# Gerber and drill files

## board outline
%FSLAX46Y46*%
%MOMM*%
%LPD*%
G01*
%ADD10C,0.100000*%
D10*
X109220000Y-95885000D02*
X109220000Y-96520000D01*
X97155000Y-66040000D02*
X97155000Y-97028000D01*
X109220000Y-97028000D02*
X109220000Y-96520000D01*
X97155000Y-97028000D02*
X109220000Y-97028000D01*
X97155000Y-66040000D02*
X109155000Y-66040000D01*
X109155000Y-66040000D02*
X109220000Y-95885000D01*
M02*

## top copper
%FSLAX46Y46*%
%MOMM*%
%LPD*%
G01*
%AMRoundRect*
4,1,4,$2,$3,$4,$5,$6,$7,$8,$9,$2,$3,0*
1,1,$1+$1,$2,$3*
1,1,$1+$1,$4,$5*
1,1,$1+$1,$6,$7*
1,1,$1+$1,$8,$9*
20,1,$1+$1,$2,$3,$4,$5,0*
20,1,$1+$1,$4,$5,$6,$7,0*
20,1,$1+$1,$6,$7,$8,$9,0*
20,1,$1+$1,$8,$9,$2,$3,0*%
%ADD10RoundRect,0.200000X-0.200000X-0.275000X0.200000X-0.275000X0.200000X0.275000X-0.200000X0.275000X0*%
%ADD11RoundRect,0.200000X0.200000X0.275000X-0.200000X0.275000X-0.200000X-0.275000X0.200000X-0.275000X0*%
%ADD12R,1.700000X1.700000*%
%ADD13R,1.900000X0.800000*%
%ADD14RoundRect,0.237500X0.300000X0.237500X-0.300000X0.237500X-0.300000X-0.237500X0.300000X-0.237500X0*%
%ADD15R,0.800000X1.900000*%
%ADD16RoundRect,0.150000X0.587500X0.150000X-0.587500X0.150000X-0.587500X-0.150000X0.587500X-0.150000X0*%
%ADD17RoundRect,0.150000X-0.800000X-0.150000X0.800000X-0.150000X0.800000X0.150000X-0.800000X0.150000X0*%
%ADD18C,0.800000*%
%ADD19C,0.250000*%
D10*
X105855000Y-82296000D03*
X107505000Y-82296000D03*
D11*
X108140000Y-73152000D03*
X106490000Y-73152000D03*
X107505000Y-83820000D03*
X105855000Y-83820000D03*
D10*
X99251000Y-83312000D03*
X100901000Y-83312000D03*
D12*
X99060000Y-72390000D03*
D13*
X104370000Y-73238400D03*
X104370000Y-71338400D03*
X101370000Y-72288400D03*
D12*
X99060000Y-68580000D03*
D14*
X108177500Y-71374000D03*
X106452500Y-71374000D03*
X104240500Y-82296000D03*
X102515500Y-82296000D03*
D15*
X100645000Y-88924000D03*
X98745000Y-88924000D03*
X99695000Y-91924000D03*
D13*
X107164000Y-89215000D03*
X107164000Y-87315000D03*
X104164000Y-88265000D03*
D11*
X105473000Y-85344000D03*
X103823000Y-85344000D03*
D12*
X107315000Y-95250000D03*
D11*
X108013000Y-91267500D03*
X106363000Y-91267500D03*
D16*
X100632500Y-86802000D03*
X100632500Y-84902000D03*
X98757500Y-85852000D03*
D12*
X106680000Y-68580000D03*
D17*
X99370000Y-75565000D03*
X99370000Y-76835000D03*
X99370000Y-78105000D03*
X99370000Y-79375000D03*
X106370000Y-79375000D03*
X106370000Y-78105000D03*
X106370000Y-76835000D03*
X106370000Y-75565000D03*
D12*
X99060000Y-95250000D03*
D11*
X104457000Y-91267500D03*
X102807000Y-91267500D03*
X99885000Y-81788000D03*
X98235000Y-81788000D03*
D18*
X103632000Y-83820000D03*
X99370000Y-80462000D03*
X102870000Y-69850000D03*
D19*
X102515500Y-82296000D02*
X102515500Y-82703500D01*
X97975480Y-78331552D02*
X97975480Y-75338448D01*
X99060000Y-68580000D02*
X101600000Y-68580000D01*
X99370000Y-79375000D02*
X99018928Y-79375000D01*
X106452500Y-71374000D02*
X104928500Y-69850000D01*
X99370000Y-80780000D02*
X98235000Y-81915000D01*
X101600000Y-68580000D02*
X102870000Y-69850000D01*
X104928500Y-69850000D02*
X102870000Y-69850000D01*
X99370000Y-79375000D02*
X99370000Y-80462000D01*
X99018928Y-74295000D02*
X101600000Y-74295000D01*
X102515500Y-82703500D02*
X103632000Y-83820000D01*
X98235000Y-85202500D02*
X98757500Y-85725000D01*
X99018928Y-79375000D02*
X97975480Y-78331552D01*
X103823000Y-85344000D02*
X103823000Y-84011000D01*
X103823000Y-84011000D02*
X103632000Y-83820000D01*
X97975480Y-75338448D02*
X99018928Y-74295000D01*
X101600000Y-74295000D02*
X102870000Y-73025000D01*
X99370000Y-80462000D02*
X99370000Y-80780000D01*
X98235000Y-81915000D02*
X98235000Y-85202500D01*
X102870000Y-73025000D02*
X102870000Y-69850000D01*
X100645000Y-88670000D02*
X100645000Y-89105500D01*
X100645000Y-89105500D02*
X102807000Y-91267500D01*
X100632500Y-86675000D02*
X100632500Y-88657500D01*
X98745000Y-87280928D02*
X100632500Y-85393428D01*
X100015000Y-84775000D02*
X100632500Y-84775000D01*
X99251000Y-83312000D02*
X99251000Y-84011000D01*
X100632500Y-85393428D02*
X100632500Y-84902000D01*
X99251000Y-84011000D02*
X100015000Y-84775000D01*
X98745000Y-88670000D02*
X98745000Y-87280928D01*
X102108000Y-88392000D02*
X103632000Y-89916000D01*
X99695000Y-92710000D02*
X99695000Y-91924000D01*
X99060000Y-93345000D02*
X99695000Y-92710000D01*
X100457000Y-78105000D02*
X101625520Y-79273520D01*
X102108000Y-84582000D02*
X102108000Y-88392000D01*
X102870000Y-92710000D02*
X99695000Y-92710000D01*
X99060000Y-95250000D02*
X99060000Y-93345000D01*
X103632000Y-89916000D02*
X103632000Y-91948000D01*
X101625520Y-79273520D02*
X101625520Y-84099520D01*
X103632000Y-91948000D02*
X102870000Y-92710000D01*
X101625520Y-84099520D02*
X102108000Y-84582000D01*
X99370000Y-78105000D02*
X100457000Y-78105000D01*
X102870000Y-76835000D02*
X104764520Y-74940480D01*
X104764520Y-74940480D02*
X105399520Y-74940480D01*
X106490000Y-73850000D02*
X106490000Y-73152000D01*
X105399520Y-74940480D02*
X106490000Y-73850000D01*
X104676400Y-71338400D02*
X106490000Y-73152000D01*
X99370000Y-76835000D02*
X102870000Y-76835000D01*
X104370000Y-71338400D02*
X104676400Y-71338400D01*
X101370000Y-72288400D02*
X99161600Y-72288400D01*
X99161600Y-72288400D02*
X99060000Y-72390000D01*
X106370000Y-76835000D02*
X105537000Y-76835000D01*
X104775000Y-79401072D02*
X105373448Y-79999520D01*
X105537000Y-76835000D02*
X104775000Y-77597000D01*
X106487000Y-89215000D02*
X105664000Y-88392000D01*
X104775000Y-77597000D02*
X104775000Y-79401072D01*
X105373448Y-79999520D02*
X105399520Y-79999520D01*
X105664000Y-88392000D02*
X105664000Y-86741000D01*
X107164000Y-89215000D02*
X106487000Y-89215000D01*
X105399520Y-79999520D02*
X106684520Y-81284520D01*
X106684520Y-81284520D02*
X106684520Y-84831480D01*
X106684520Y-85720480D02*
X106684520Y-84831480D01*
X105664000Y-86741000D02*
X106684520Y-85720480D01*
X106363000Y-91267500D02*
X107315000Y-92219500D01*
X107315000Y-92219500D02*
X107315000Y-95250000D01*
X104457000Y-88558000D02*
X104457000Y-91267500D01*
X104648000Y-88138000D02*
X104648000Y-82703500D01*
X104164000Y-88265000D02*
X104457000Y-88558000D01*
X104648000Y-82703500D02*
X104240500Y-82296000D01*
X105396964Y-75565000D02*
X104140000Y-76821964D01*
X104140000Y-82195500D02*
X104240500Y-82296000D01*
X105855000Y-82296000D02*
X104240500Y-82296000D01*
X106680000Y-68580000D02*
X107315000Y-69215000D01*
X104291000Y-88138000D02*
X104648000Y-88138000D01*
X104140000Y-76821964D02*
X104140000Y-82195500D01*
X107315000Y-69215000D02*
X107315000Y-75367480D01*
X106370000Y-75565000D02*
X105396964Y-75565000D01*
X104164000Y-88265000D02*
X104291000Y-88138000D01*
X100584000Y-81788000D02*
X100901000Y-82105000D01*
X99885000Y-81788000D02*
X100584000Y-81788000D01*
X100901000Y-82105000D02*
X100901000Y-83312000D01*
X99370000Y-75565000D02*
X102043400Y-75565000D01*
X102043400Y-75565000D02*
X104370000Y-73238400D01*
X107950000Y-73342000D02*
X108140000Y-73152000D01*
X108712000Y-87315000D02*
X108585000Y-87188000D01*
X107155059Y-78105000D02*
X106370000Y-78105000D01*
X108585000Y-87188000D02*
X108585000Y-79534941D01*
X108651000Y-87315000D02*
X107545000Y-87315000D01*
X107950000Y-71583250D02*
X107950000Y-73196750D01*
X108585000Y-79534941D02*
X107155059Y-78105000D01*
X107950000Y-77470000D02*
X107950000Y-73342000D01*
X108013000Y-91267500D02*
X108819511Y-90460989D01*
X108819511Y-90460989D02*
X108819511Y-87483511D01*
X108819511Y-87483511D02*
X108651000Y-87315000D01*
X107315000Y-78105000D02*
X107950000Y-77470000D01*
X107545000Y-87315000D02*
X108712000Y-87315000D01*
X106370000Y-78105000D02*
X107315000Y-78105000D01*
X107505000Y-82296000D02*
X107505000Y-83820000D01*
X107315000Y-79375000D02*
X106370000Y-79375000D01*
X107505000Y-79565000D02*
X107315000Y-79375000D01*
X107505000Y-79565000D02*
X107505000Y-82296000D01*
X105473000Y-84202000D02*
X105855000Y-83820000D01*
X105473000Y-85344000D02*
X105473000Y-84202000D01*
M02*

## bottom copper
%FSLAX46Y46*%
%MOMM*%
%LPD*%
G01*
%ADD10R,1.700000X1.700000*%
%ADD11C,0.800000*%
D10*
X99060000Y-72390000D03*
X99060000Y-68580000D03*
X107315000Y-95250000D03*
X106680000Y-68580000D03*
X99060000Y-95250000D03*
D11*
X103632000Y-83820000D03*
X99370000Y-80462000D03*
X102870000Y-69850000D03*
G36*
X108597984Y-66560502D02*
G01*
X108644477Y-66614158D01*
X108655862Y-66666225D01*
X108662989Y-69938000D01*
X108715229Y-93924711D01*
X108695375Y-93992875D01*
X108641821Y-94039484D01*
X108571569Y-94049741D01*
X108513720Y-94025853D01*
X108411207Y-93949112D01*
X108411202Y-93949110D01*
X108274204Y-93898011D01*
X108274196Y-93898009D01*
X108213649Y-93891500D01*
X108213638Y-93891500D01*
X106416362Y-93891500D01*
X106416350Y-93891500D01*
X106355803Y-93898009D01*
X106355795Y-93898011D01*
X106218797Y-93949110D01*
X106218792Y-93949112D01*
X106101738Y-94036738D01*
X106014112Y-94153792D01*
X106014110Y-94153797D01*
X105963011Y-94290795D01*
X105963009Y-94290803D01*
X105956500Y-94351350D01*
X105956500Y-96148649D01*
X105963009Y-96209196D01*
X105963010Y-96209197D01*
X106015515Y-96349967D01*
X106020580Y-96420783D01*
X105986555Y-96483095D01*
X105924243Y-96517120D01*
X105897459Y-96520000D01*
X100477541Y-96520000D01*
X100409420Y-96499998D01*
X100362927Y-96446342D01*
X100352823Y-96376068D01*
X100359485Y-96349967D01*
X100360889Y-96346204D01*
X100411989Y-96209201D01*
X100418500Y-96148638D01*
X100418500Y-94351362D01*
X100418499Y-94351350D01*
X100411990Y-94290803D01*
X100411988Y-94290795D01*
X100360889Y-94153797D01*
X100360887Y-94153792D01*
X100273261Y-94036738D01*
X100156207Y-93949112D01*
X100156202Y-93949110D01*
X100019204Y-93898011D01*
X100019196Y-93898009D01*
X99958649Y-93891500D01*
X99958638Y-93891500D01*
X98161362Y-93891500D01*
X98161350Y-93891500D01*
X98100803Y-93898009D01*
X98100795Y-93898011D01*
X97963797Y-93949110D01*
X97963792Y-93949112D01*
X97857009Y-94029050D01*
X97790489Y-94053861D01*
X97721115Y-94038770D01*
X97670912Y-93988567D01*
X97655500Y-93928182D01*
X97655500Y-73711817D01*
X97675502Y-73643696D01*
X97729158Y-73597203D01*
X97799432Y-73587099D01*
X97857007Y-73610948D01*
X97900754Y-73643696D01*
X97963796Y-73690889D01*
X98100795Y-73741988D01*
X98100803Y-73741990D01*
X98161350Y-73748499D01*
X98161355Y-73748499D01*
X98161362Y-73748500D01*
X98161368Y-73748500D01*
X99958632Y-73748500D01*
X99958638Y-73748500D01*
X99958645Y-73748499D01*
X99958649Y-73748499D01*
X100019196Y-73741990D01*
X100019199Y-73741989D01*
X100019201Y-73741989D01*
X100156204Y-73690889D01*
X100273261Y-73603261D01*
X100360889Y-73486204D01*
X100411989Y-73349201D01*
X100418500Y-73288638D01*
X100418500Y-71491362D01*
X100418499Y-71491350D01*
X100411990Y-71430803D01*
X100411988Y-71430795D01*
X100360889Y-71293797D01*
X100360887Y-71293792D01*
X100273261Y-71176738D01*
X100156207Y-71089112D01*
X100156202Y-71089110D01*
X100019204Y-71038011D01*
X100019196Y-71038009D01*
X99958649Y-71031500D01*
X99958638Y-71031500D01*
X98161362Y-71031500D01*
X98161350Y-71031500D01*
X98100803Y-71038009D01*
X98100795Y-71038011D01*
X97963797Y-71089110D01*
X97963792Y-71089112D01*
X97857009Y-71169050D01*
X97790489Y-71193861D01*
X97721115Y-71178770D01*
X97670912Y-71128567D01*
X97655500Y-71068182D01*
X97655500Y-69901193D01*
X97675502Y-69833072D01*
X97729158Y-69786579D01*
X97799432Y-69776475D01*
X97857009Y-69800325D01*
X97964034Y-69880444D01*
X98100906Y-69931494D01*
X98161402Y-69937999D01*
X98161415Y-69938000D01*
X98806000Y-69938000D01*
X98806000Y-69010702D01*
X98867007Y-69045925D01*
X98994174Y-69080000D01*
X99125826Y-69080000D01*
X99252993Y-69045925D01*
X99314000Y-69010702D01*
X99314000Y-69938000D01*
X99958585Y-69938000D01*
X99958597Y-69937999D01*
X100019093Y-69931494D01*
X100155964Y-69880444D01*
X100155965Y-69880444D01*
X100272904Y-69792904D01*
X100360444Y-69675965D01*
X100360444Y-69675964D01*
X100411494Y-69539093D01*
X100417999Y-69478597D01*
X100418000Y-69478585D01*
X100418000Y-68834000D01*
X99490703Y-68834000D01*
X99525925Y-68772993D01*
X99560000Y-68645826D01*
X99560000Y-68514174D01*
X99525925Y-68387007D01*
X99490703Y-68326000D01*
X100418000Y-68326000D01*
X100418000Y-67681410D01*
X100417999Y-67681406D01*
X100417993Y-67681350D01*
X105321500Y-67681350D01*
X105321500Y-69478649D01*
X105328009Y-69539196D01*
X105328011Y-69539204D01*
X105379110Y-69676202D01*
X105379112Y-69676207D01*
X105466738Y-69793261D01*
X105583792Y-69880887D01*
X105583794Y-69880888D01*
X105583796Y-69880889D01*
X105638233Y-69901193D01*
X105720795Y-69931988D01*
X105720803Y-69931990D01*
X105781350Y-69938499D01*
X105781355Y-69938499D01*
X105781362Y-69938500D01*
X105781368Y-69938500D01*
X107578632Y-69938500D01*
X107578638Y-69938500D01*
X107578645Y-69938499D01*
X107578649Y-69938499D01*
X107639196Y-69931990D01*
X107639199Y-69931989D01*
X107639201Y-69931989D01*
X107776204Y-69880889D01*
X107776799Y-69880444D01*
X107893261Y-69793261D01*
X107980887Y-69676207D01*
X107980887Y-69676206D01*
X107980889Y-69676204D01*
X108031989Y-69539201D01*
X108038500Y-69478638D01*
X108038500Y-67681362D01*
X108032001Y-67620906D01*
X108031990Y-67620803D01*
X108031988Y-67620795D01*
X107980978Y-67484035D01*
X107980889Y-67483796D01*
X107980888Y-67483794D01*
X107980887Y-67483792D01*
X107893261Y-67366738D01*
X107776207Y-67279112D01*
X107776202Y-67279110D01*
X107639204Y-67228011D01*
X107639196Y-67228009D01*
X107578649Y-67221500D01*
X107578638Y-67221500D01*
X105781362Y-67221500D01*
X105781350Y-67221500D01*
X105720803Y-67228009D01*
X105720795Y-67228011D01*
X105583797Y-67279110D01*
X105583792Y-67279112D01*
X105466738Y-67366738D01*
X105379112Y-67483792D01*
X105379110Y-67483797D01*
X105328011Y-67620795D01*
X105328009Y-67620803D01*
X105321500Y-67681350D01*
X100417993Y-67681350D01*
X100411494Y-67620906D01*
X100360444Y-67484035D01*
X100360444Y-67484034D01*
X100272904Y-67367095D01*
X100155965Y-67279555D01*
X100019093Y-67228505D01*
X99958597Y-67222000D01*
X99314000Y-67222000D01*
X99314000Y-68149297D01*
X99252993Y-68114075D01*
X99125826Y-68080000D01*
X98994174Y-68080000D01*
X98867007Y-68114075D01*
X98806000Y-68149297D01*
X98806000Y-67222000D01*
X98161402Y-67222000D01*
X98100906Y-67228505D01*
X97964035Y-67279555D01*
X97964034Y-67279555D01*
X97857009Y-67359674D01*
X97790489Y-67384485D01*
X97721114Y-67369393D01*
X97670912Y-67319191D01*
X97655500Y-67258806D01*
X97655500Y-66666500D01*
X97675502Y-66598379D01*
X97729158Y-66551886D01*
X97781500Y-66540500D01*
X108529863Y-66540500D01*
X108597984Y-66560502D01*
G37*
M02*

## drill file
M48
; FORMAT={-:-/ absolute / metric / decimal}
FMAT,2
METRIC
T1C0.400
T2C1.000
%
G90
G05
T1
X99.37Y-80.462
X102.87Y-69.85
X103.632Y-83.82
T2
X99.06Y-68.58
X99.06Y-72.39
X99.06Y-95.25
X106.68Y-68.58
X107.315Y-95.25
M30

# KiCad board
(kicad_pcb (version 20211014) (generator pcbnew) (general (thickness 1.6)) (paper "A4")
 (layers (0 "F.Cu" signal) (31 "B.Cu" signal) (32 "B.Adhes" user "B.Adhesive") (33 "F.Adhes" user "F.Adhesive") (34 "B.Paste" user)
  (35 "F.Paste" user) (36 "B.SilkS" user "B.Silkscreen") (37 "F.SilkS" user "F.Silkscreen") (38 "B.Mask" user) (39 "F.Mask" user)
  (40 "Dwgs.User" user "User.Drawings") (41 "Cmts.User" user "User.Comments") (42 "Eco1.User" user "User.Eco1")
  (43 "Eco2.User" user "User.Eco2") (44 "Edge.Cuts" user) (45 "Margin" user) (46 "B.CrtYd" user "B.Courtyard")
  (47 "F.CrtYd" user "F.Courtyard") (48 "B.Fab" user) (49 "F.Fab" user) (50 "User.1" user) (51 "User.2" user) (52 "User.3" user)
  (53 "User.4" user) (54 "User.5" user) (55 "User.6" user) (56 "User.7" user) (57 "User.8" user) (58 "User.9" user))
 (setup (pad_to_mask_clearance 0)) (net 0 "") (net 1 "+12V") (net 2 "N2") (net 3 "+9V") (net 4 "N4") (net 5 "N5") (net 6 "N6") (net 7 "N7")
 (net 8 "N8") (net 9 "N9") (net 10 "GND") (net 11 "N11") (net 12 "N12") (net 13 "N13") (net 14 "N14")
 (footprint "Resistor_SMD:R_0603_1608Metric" (layer "F.Cu") (at 106.68 82.296)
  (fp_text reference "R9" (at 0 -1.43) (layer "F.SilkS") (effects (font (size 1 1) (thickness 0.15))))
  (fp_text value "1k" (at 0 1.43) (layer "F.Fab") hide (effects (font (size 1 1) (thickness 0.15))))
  (pad "1" smd roundrect (at -0.825 0) (size 0.8 0.95) (layers "F.Cu" "F.Paste" "F.Mask") (roundrect_rratio 0.25) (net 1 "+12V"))
  (pad "2" smd roundrect (at 0.825 0) (size 0.8 0.95) (layers "F.Cu" "F.Paste" "F.Mask") (roundrect_rratio 0.25) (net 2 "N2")))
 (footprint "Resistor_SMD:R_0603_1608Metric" (layer "F.Cu") (at 107.315 73.152 180)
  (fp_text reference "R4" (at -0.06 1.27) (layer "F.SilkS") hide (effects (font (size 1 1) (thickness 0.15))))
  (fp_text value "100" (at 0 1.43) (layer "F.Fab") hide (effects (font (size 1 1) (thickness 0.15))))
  (pad "1" smd roundrect (at -0.825 0 180) (size 0.8 0.95) (layers "F.Cu" "F.Paste" "F.Mask") (roundrect_rratio 0.25) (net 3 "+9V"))
  (pad "2" smd roundrect (at 0.825 0 180) (size 0.8 0.95) (layers "F.Cu" "F.Paste" "F.Mask") (roundrect_rratio 0.25) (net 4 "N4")))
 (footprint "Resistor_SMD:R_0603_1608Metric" (layer "F.Cu") (at 106.68 83.82 180)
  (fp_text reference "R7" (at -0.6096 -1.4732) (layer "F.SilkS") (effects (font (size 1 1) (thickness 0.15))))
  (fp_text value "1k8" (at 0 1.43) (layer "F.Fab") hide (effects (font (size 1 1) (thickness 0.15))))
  (pad "1" smd roundrect (at -0.825 0 180) (size 0.8 0.95) (layers "F.Cu" "F.Paste" "F.Mask") (roundrect_rratio 0.25) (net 2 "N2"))
  (pad "2" smd roundrect (at 0.825 0 180) (size 0.8 0.95) (layers "F.Cu" "F.Paste" "F.Mask") (roundrect_rratio 0.25) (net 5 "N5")))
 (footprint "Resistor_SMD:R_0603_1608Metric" (layer "F.Cu") (at 100.076 83.312)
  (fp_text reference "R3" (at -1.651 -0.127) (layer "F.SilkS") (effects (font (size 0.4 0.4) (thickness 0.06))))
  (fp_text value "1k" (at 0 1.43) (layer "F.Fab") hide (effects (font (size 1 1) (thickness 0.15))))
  (pad "1" smd roundrect (at -0.825 0) (size 0.8 0.95) (layers "F.Cu" "F.Paste" "F.Mask") (roundrect_rratio 0.25) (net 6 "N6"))
  (pad "2" smd roundrect (at 0.825 0) (size 0.8 0.95) (layers "F.Cu" "F.Paste" "F.Mask") (roundrect_rratio 0.25) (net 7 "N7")))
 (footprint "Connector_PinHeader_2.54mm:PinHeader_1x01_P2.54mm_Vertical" (layer "F.Cu") (at 99.06 72.39)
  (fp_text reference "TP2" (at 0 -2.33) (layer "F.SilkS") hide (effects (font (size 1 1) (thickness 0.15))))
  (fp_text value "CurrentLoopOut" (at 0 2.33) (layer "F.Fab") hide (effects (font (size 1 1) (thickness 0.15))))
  (pad "1" thru_hole rect (at 0 0) (size 1.7 1.7) (drill 1) (layers *.Cu *.Mask) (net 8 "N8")))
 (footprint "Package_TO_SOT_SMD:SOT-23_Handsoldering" (layer "F.Cu") (at 102.87 72.2884 180)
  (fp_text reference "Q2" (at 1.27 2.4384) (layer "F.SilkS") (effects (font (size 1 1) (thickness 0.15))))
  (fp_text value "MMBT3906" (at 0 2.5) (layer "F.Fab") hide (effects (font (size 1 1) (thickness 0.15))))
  (pad "1" smd rect (at -1.5 -0.95 180) (size 1.9 0.8) (layers "F.Cu" "F.Paste" "F.Mask") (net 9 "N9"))
  (pad "2" smd rect (at -1.5 0.95 180) (size 1.9 0.8) (layers "F.Cu" "F.Paste" "F.Mask") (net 4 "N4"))
  (pad "3" smd rect (at 1.5 0 180) (size 1.9 0.8) (layers "F.Cu" "F.Paste" "F.Mask") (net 8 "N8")))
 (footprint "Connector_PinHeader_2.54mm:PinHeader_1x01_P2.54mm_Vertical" (layer "F.Cu") (at 99.06 68.58)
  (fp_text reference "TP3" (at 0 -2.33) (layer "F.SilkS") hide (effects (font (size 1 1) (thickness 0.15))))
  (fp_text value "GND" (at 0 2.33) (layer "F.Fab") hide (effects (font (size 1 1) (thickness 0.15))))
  (pad "1" thru_hole rect (at 0 0) (size 1.7 1.7) (drill 1) (layers *.Cu *.Mask) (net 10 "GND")))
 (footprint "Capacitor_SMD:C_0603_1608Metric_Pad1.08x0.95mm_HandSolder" (layer "F.Cu") (at 107.315 71.374 180)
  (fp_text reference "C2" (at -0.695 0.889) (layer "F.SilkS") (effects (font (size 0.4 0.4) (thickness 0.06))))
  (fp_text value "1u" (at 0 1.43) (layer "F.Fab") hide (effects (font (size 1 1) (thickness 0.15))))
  (pad "1" smd roundrect (at -0.8625 0 180) (size 1.075 0.95) (layers "F.Cu" "F.Paste" "F.Mask") (roundrect_rratio 0.25) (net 3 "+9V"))
  (pad "2" smd roundrect (at 0.8625 0 180) (size 1.075 0.95) (layers "F.Cu" "F.Paste" "F.Mask") (roundrect_rratio 0.25) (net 10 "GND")))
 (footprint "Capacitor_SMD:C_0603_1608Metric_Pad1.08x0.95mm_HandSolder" (layer "F.Cu") (at 103.378 82.296 180)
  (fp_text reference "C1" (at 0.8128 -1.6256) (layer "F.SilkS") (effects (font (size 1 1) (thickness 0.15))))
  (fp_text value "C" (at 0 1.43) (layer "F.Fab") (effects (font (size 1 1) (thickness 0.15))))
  (pad "1" smd roundrect (at -0.8625 0 180) (size 1.075 0.95) (layers "F.Cu" "F.Paste" "F.Mask") (roundrect_rratio 0.25) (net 1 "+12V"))
  (pad "2" smd roundrect (at 0.8625 0 180) (size 1.075 0.95) (layers "F.Cu" "F.Paste" "F.Mask") (roundrect_rratio 0.25) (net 10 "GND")))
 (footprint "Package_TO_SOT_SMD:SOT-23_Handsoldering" (layer "F.Cu") (at 99.695 90.424 -90)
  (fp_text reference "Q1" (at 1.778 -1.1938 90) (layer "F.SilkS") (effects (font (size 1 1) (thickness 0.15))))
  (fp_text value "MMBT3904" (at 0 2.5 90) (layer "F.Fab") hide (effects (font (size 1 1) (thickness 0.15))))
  (pad "1" smd rect (at -1.5 -0.95 270) (size 1.9 0.8) (layers "F.Cu" "F.Paste" "F.Mask") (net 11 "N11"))
  (pad "2" smd rect (at -1.5 0.95 270) (size 1.9 0.8) (layers "F.Cu" "F.Paste" "F.Mask") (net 6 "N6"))
  (pad "3" smd rect (at 1.5 0 270) (size 1.9 0.8) (layers "F.Cu" "F.Paste" "F.Mask") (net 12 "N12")))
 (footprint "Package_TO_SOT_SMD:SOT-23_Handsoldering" (layer "F.Cu") (at 105.664 88.265 180)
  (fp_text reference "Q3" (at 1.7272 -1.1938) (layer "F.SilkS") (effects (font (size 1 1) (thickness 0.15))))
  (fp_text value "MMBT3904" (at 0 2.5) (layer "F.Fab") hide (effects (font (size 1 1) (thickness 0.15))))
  (pad "1" smd rect (at -1.5 -0.95 180) (size 1.9 0.8) (layers "F.Cu" "F.Paste" "F.Mask") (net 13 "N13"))
  (pad "2" smd rect (at -1.5 0.95 180) (size 1.9 0.8) (layers "F.Cu" "F.Paste" "F.Mask") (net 3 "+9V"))
  (pad "3" smd rect (at 1.5 0 180) (size 1.9 0.8) (layers "F.Cu" "F.Paste" "F.Mask") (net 1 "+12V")))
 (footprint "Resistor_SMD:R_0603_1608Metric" (layer "F.Cu") (at 104.648 85.344 180)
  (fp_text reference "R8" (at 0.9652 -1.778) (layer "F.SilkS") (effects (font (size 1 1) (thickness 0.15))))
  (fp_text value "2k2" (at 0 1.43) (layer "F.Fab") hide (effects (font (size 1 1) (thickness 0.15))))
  (pad "1" smd roundrect (at -0.825 0 180) (size 0.8 0.95) (layers "F.Cu" "F.Paste" "F.Mask") (roundrect_rratio 0.25) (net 5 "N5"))
  (pad "2" smd roundrect (at 0.825 0 180) (size 0.8 0.95) (layers "F.Cu" "F.Paste" "F.Mask") (roundrect_rratio 0.25) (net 10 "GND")))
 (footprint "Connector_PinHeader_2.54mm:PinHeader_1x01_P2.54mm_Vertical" (layer "F.Cu") (at 107.315 95.25 180)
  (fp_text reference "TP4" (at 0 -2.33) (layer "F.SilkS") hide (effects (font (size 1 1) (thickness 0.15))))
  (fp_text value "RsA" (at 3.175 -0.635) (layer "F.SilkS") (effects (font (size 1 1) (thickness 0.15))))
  (pad "1" thru_hole rect (at 0 0 180) (size 1.7 1.7) (drill 1) (layers *.Cu *.Mask) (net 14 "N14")))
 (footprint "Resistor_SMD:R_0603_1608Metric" (layer "F.Cu") (at 107.188 91.2675 180)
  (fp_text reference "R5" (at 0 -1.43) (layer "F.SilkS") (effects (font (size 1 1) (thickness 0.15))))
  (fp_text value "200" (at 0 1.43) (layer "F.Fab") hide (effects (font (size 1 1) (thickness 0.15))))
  (pad "1" smd roundrect (at -0.825 0 180) (size 0.8 0.95) (layers "F.Cu" "F.Paste" "F.Mask") (roundrect_rratio 0.25) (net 3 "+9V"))
  (pad "2" smd roundrect (at 0.825 0 180) (size 0.8 0.95) (layers "F.Cu" "F.Paste" "F.Mask") (roundrect_rratio 0.25) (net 14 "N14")))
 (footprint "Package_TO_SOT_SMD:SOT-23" (layer "F.Cu") (at 99.695 85.852 180)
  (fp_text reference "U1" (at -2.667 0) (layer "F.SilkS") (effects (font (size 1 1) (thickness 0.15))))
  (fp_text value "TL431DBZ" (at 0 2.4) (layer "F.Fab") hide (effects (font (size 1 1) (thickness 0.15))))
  (pad "1" smd roundrect (at -0.9375 -0.95 180) (size 1.475 0.6) (layers "F.Cu" "F.Paste" "F.Mask") (roundrect_rratio 0.25) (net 11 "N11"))
  (pad "2" smd roundrect (at -0.9375 0.95 180) (size 1.475 0.6) (layers "F.Cu" "F.Paste" "F.Mask") (roundrect_rratio 0.25) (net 6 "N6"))
  (pad "3" smd roundrect (at 0.9375 0 180) (size 1.475 0.6) (layers "F.Cu" "F.Paste" "F.Mask") (roundrect_rratio 0.25) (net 10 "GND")))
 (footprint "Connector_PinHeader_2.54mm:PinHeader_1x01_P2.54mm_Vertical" (layer "F.Cu") (at 106.68 68.58)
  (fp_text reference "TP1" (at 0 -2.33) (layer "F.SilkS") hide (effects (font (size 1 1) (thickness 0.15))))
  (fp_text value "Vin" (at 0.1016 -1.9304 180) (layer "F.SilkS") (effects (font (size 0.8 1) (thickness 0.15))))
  (pad "1" thru_hole rect (at 0 0) (size 1.7 1.7) (drill 1) (layers *.Cu *.Mask) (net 1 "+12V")))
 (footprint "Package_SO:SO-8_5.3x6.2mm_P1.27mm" (layer "F.Cu") (at 102.87 77.47)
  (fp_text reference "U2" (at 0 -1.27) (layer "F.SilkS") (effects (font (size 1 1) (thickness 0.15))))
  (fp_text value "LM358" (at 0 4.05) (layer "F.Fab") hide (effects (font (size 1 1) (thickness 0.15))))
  (pad "1" smd roundrect (at -3.5 -1.905) (size 1.9 0.6) (layers "F.Cu" "F.Paste" "F.Mask") (roundrect_rratio 0.25) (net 9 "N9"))
  (pad "2" smd roundrect (at -3.5 -0.635) (size 1.9 0.6) (layers "F.Cu" "F.Paste" "F.Mask") (roundrect_rratio 0.25) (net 4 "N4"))
  (pad "3" smd roundrect (at -3.5 0.635) (size 1.9 0.6) (layers "F.Cu" "F.Paste" "F.Mask") (roundrect_rratio 0.25) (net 12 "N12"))
  (pad "4" smd roundrect (at -3.5 1.905) (size 1.9 0.6) (layers "F.Cu" "F.Paste" "F.Mask") (roundrect_rratio 0.25) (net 10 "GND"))
  (pad "5" smd roundrect (at 3.5 1.905) (size 1.9 0.6) (layers "F.Cu" "F.Paste" "F.Mask") (roundrect_rratio 0.25) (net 2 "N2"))
  (pad "6" smd roundrect (at 3.5 0.635) (size 1.9 0.6) (layers "F.Cu" "F.Paste" "F.Mask") (roundrect_rratio 0.25) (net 3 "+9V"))
  (pad "7" smd roundrect (at 3.5 -0.635) (size 1.9 0.6) (layers "F.Cu" "F.Paste" "F.Mask") (roundrect_rratio 0.25) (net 13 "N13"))
  (pad "8" smd roundrect (at 3.5 -1.905) (size 1.9 0.6) (layers "F.Cu" "F.Paste" "F.Mask") (roundrect_rratio 0.25) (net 1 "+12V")))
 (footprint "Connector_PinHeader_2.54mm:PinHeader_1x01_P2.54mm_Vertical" (layer "F.Cu") (at 99.06 95.25 180)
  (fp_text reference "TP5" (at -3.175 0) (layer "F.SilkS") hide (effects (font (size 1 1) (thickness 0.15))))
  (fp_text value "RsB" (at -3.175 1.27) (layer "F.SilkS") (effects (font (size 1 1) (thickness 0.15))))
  (pad "1" thru_hole rect (at 0 0 180) (size 1.7 1.7) (drill 1) (layers *.Cu *.Mask) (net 12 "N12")))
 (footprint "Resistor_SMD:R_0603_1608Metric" (layer "F.Cu") (at 103.632 91.2675 180)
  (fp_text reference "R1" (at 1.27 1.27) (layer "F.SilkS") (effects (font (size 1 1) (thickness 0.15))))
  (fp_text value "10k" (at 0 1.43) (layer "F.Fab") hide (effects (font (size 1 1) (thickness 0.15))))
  (pad "1" smd roundrect (at -0.825 0 180) (size 0.8 0.95) (layers "F.Cu" "F.Paste" "F.Mask") (roundrect_rratio 0.25) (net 1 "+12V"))
  (pad "2" smd roundrect (at 0.825 0 180) (size 0.8 0.95) (layers "F.Cu" "F.Paste" "F.Mask") (roundrect_rratio 0.25) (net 11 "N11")))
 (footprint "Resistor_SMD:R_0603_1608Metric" (layer "F.Cu") (at 99.06 81.788 180)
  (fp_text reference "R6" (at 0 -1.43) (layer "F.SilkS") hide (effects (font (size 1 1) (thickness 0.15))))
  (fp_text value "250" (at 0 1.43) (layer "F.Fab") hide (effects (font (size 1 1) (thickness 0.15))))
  (pad "1" smd roundrect (at -0.825 0 180) (size 0.8 0.95) (layers "F.Cu" "F.Paste" "F.Mask") (roundrect_rratio 0.25) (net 7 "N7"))
  (pad "2" smd roundrect (at 0.825 0 180) (size 0.8 0.95) (layers "F.Cu" "F.Paste" "F.Mask") (roundrect_rratio 0.25) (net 10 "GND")))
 (gr_line (start 109.22 95.885) (end 109.22 96.52) (layer "Edge.Cuts") (width 0.1))
 (gr_line (start 97.155 66.04) (end 97.155 97.028) (layer "Edge.Cuts") (width 0.1))
 (gr_line (start 109.22 97.028) (end 109.22 96.52) (layer "Edge.Cuts") (width 0.1))
 (gr_line (start 97.155 97.028) (end 109.22 97.028) (layer "Edge.Cuts") (width 0.1))
 (gr_line (start 97.155 66.04) (end 109.155 66.04) (layer "Edge.Cuts") (width 0.1))
 (gr_line (start 109.155 66.04) (end 109.22 95.885) (layer "Edge.Cuts") (width 0.1))
 (segment (start 102.5155 82.296) (end 102.5155 82.7035) (width 0.25) (layer "F.Cu") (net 10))
 (segment (start 97.97548 78.331552) (end 97.97548 75.338448) (width 0.25) (layer "F.Cu") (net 10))
 (segment (start 99.06 68.58) (end 101.6 68.58) (width 0.25) (layer "F.Cu") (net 10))
 (segment (start 99.37 79.375) (end 99.018928 79.375) (width 0.25) (layer "F.Cu") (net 10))
 (segment (start 106.4525 71.374) (end 104.9285 69.85) (width 0.25) (layer "F.Cu") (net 10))
 (segment (start 99.37 80.78) (end 98.235 81.915) (width 0.25) (layer "F.Cu") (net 10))
 (segment (start 101.6 68.58) (end 102.87 69.85) (width 0.25) (layer "F.Cu") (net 10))
 (segment (start 104.9285 69.85) (end 102.87 69.85) (width 0.25) (layer "F.Cu") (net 10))
 (segment (start 99.37 79.375) (end 99.37 80.462) (width 0.25) (layer "F.Cu") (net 10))
 (segment (start 99.018928 74.295) (end 101.6 74.295) (width 0.25) (layer "F.Cu") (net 10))
 (segment (start 102.5155 82.7035) (end 103.632 83.82) (width 0.25) (layer "F.Cu") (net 10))
 (segment (start 98.235 85.2025) (end 98.7575 85.725) (width 0.25) (layer "F.Cu") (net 10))
 (segment (start 99.018928 79.375) (end 97.97548 78.331552) (width 0.25) (layer "F.Cu") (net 10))
 (segment (start 103.823 85.344) (end 103.823 84.011) (width 0.25) (layer "F.Cu") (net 10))
 (segment (start 103.823 84.011) (end 103.632 83.82) (width 0.25) (layer "F.Cu") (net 10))
 (segment (start 97.97548 75.338448) (end 99.018928 74.295) (width 0.25) (layer "F.Cu") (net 10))
 (segment (start 101.6 74.295) (end 102.87 73.025) (width 0.25) (layer "F.Cu") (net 10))
 (segment (start 99.37 80.462) (end 99.37 80.78) (width 0.25) (layer "F.Cu") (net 10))
 (segment (start 98.235 81.915) (end 98.235 85.2025) (width 0.25) (layer "F.Cu") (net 10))
 (segment (start 102.87 73.025) (end 102.87 69.85) (width 0.25) (layer "F.Cu") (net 10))
 (via (at 103.632 83.82) (size 0.8) (drill 0.4) (layers "F.Cu" "B.Cu") (free) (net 10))
 (via (at 99.37 80.462) (size 0.8) (drill 0.4) (layers "F.Cu" "B.Cu") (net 10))
 (via (at 102.87 69.85) (size 0.8) (drill 0.4) (layers "F.Cu" "B.Cu") (free) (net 10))
 (segment (start 100.645 88.67) (end 100.645 89.1055) (width 0.25) (layer "F.Cu") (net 11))
 (segment (start 100.645 89.1055) (end 102.807 91.2675) (width 0.25) (layer "F.Cu") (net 11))
 (segment (start 100.6325 86.675) (end 100.6325 88.6575) (width 0.25) (layer "F.Cu") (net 11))
 (segment (start 98.745 87.280928) (end 100.6325 85.393428) (width 0.25) (layer "F.Cu") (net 6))
 (segment (start 100.015 84.775) (end 100.6325 84.775) (width 0.25) (layer "F.Cu") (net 6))
 (segment (start 99.251 83.312) (end 99.251 84.011) (width 0.25) (layer "F.Cu") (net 6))
 (segment (start 100.6325 85.393428) (end 100.6325 84.902) (width 0.25) (layer "F.Cu") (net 6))
 (segment (start 99.251 84.011) (end 100.015 84.775) (width 0.25) (layer "F.Cu") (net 6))
 (segment (start 98.745 88.67) (end 98.745 87.280928) (width 0.25) (layer "F.Cu") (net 6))
 (segment (start 102.108 88.392) (end 103.632 89.916) (width 0.25) (layer "F.Cu") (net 12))
 (segment (start 99.695 92.71) (end 99.695 91.924) (width 0.25) (layer "F.Cu") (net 12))
 (segment (start 99.06 93.345) (end 99.695 92.71) (width 0.25) (layer "F.Cu") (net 12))
 (segment (start 100.457 78.105) (end 101.62552 79.27352) (width 0.25) (layer "F.Cu") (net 12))
 (segment (start 102.108 84.582) (end 102.108 88.392) (width 0.25) (layer "F.Cu") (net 12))
 (segment (start 102.87 92.71) (end 99.695 92.71) (width 0.25) (layer "F.Cu") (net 12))
 (segment (start 99.06 95.25) (end 99.06 93.345) (width 0.25) (layer "F.Cu") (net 12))
 (segment (start 103.632 89.916) (end 103.632 91.948) (width 0.25) (layer "F.Cu") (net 12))
 (segment (start 101.62552 79.27352) (end 101.62552 84.09952) (width 0.25) (layer "F.Cu") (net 12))
 (segment (start 103.632 91.948) (end 102.87 92.71) (width 0.25) (layer "F.Cu") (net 12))
 (segment (start 101.62552 84.09952) (end 102.108 84.582) (width 0.25) (layer "F.Cu") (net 12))
 (segment (start 99.37 78.105) (end 100.457 78.105) (width 0.25) (layer "F.Cu") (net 12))
 (segment (start 102.87 76.835) (end 104.76452 74.94048) (width 0.25) (layer "F.Cu") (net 4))
 (segment (start 104.76452 74.94048) (end 105.39952 74.94048) (width 0.25) (layer "F.Cu") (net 4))
 (segment (start 106.49 73.85) (end 106.49 73.152) (width 0.25) (layer "F.Cu") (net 4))
 (segment (start 105.39952 74.94048) (end 106.49 73.85) (width 0.25) (layer "F.Cu") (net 4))
 (segment (start 104.6764 71.3384) (end 106.49 73.152) (width 0.25) (layer "F.Cu") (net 4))
 (segment (start 99.37 76.835) (end 102.87 76.835) (width 0.25) (layer "F.Cu") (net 4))
 (segment (start 104.37 71.3384) (end 104.6764 71.3384) (width 0.25) (layer "F.Cu") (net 4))
 (segment (start 101.37 72.2884) (end 99.1616 72.2884) (width 0.25) (layer "F.Cu") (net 8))
 (segment (start 99.1616 72.2884) (end 99.06 72.39) (width 0.25) (layer "F.Cu") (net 8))
 (segment (start 106.37 76.835) (end 105.537 76.835) (width 0.25) (layer "F.Cu") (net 13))
 (segment (start 104.775 79.401072) (end 105.373448 79.99952) (width 0.25) (layer "F.Cu") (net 13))
 (segment (start 105.537 76.835) (end 104.775 77.597) (width 0.25) (layer "F.Cu") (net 13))
 (segment (start 106.487 89.215) (end 105.664 88.392) (width 0.25) (layer "F.Cu") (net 13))
 (segment (start 104.775 77.597) (end 104.775 79.401072) (width 0.25) (layer "F.Cu") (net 13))
 (segment (start 105.373448 79.99952) (end 105.39952 79.99952) (width 0.25) (layer "F.Cu") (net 13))
 (segment (start 105.664 88.392) (end 105.664 86.741) (width 0.25) (layer "F.Cu") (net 13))
 (segment (start 107.164 89.215) (end 106.487 89.215) (width 0.25) (layer "F.Cu") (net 13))
 (segment (start 105.39952 79.99952) (end 106.68452 81.28452) (width 0.25) (layer "F.Cu") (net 13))
 (segment (start 106.68452 81.28452) (end 106.68452 84.83148) (width 0.25) (layer "F.Cu") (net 13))
 (segment (start 106.68452 85.72048) (end 106.68452 84.83148) (width 0.25) (layer "F.Cu") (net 13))
 (segment (start 105.664 86.741) (end 106.68452 85.72048) (width 0.25) (layer "F.Cu") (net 13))
 (segment (start 106.363 91.2675) (end 107.315 92.2195) (width 0.25) (layer "F.Cu") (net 14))
 (segment (start 107.315 92.2195) (end 107.315 95.25) (width 0.25) (layer "F.Cu") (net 14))
 (segment (start 104.457 88.558) (end 104.457 91.2675) (width 0.25) (layer "F.Cu") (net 1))
 (segment (start 104.648 88.138) (end 104.648 82.7035) (width 0.25) (layer "F.Cu") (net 1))
 (segment (start 104.164 88.265) (end 104.457 88.558) (width 0.25) (layer "F.Cu") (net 1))
 (segment (start 104.648 82.7035) (end 104.2405 82.296) (width 0.25) (layer "F.Cu") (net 1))
 (segment (start 105.396964 75.565) (end 104.14 76.821964) (width 0.25) (layer "F.Cu") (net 1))
 (segment (start 104.14 82.1955) (end 104.2405 82.296) (width 0.25) (layer "F.Cu") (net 1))
 (segment (start 105.855 82.296) (end 104.2405 82.296) (width 0.25) (layer "F.Cu") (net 1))
 (segment (start 106.68 68.58) (end 107.315 69.215) (width 0.25) (layer "F.Cu") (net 1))
 (segment (start 104.291 88.138) (end 104.648 88.138) (width 0.25) (layer "F.Cu") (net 1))
 (segment (start 104.14 76.821964) (end 104.14 82.1955) (width 0.25) (layer "F.Cu") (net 1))
 (segment (start 107.315 69.215) (end 107.315 75.36748) (width 0.25) (layer "F.Cu") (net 1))
 (segment (start 106.37 75.565) (end 105.396964 75.565) (width 0.25) (layer "F.Cu") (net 1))
 (segment (start 104.164 88.265) (end 104.291 88.138) (width 0.25) (layer "F.Cu") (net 1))
 (segment (start 100.584 81.788) (end 100.901 82.105) (width 0.25) (layer "F.Cu") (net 7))
 (segment (start 99.885 81.788) (end 100.584 81.788) (width 0.25) (layer "F.Cu") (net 7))
 (segment (start 100.901 82.105) (end 100.901 83.312) (width 0.25) (layer "F.Cu") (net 7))
 (segment (start 99.37 75.565) (end 102.0434 75.565) (width 0.25) (layer "F.Cu") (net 9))
 (segment (start 102.0434 75.565) (end 104.37 73.2384) (width 0.25) (layer "F.Cu") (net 9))
 (segment (start 107.95 73.342) (end 108.14 73.152) (width 0.25) (layer "F.Cu") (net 3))
 (segment (start 108.712 87.315) (end 108.585 87.188) (width 0.25) (layer "F.Cu") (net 3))
 (segment (start 107.155059 78.105) (end 106.37 78.105) (width 0.25) (layer "F.Cu") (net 3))
 (segment (start 108.585 87.188) (end 108.585 79.534941) (width 0.25) (layer "F.Cu") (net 3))
 (segment (start 108.651 87.315) (end 107.545 87.315) (width 0.25) (layer "F.Cu") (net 3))
 (segment (start 107.95 71.58325) (end 107.95 73.19675) (width 0.25) (layer "F.Cu") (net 3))
 (segment (start 108.585 79.534941) (end 107.155059 78.105) (width 0.25) (layer "F.Cu") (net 3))
 (segment (start 107.95 77.47) (end 107.95 73.342) (width 0.25) (layer "F.Cu") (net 3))
 (segment (start 108.013 91.2675) (end 108.819511 90.460989) (width 0.25) (layer "F.Cu") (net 3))
 (segment (start 108.819511 90.460989) (end 108.819511 87.483511) (width 0.25) (layer "F.Cu") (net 3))
 (segment (start 108.819511 87.483511) (end 108.651 87.315) (width 0.25) (layer "F.Cu") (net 3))
 (segment (start 107.315 78.105) (end 107.95 77.47) (width 0.25) (layer "F.Cu") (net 3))
 (segment (start 107.545 87.315) (end 108.712 87.315) (width 0.25) (layer "F.Cu") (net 3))
 (segment (start 106.37 78.105) (end 107.315 78.105) (width 0.25) (layer "F.Cu") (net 3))
 (segment (start 107.505 82.296) (end 107.505 83.82) (width 0.25) (layer "F.Cu") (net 2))
 (segment (start 107.315 79.375) (end 106.37 79.375) (width 0.25) (layer "F.Cu") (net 2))
 (segment (start 107.505 79.565) (end 107.315 79.375) (width 0.25) (layer "F.Cu") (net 2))
 (segment (start 107.505 79.565) (end 107.505 82.296) (width 0.25) (layer "F.Cu") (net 2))
 (segment (start 105.473 84.202) (end 105.855 83.82) (width 0.25) (layer "F.Cu") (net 5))
 (segment (start 105.473 85.344) (end 105.473 84.202) (width 0.25) (layer "F.Cu") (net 5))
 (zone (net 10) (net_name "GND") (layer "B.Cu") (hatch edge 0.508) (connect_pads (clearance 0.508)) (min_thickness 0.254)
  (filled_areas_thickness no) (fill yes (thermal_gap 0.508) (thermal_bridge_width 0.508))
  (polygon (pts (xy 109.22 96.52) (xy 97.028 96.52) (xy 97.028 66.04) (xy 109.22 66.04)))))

